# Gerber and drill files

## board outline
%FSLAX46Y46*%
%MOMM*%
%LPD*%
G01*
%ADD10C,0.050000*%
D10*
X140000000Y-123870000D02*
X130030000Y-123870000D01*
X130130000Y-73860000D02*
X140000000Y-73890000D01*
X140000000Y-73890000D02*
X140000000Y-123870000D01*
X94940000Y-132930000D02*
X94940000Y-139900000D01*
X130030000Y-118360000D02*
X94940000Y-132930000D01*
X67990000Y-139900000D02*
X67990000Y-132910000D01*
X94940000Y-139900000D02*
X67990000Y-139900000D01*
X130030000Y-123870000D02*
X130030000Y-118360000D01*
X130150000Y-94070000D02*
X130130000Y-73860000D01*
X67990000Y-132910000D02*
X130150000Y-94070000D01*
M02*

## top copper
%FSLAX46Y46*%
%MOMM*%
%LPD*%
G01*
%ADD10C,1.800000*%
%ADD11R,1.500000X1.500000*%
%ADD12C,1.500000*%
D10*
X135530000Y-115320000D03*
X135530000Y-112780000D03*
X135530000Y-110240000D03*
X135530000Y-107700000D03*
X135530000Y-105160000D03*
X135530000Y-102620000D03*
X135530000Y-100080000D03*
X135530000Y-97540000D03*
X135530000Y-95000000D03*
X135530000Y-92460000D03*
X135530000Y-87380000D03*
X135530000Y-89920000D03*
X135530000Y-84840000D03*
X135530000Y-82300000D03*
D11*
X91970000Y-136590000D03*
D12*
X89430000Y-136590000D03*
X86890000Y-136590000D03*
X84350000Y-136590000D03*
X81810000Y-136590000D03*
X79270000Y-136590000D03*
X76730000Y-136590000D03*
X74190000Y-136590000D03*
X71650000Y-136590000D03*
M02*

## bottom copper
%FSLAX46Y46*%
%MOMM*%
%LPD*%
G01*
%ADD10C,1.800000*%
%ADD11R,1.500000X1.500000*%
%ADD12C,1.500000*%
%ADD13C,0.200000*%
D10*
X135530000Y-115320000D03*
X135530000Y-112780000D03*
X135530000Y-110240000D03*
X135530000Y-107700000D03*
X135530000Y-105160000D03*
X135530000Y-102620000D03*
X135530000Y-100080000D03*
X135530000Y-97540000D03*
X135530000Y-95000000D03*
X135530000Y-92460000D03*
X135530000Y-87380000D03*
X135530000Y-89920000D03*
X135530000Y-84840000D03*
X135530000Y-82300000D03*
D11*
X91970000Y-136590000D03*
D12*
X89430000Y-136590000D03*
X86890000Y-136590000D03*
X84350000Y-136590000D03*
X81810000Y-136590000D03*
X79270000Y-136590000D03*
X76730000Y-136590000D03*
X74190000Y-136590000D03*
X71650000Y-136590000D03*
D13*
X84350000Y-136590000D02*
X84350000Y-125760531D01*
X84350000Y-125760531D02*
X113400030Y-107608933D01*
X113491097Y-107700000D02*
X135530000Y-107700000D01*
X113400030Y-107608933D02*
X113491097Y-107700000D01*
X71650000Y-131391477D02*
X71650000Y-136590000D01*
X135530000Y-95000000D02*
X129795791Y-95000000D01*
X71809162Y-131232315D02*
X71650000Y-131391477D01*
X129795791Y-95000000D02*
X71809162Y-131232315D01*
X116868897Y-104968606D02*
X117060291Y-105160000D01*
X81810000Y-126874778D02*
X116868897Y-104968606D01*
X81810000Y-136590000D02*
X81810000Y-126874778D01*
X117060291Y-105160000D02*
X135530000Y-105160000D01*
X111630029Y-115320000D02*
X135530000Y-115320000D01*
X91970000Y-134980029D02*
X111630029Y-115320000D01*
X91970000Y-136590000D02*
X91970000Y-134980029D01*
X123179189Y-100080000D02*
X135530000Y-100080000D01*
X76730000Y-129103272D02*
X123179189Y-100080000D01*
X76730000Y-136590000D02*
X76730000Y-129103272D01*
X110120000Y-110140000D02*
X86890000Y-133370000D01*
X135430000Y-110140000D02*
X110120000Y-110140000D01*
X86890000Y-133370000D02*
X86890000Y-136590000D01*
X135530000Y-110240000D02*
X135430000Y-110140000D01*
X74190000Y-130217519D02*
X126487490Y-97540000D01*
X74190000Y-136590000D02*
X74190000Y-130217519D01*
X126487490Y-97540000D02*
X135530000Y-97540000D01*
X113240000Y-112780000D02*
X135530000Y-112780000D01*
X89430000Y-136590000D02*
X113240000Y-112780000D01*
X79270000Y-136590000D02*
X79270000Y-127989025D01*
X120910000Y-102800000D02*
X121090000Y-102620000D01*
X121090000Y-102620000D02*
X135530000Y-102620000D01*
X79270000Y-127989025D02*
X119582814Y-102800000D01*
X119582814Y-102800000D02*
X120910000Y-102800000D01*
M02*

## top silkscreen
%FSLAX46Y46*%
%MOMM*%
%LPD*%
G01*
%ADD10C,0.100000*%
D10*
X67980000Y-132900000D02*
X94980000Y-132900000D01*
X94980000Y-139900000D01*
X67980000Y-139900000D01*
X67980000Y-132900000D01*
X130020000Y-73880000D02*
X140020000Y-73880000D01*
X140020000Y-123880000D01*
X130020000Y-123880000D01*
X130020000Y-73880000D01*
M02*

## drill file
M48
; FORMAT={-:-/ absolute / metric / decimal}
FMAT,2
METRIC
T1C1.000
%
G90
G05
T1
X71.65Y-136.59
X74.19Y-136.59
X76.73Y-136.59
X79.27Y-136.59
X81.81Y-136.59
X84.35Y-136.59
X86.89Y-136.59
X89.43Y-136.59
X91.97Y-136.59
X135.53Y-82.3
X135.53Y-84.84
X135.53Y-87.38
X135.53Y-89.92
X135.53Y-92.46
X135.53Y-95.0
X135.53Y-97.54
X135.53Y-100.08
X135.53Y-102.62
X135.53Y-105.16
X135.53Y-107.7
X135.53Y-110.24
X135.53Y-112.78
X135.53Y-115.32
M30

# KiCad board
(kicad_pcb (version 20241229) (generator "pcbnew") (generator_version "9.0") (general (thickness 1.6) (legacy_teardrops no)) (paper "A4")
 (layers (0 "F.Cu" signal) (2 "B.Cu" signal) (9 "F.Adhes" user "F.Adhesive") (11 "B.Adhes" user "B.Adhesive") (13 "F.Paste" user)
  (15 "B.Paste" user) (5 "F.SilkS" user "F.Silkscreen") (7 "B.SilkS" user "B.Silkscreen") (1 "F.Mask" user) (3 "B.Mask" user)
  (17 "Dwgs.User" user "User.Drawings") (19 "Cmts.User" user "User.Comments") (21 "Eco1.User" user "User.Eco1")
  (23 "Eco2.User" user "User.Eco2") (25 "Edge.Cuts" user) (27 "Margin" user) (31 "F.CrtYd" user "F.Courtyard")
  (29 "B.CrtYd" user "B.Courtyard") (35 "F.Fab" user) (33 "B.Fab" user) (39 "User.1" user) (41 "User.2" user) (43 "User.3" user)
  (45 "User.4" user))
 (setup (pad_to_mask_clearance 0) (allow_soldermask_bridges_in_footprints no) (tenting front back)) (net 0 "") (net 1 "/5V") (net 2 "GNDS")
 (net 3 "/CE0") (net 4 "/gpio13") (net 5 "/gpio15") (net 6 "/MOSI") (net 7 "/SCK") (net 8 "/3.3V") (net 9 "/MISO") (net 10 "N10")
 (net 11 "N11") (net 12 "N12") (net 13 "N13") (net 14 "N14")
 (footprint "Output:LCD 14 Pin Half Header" (layer "F.Cu") (at 133.02 73.88)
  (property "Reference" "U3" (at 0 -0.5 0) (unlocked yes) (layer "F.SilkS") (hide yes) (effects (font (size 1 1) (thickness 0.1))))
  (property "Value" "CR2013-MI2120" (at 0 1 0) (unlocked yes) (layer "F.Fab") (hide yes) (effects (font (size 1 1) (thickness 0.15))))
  (fp_rect (start -3 0) (end 7 50) (stroke (width 0.1) (type solid)) (fill no) (layer "F.SilkS"))
  (pad "1" thru_hole circle (at 2.51 41.44 180) (size 1.8 1.8) (drill 1) (layers "*.Cu" "*.Mask") (remove_unused_layers no) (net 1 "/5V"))
  (pad "2" thru_hole circle (at 2.51 38.9 180) (size 1.8 1.8) (drill 1) (layers "*.Cu" "*.Mask") (remove_unused_layers no) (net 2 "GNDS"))
  (pad "3" thru_hole circle (at 2.51 36.36 180) (size 1.8 1.8) (drill 1) (layers "*.Cu" "*.Mask") (remove_unused_layers no) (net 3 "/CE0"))
  (pad "4" thru_hole circle (at 2.51 33.82 180) (size 1.8 1.8) (drill 1) (layers "*.Cu" "*.Mask") (remove_unused_layers no)
   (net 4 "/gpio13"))
  (pad "5" thru_hole circle (at 2.51 31.28 180) (size 1.8 1.8) (drill 1) (layers "*.Cu" "*.Mask") (remove_unused_layers no)
   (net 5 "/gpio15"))
  (pad "6" thru_hole circle (at 2.51 28.74 180) (size 1.8 1.8) (drill 1) (layers "*.Cu" "*.Mask") (remove_unused_layers no) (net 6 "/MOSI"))
  (pad "7" thru_hole circle (at 2.51 26.2 180) (size 1.8 1.8) (drill 1) (layers "*.Cu" "*.Mask") (remove_unused_layers no) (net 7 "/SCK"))
  (pad "8" thru_hole circle (at 2.51 23.66 180) (size 1.8 1.8) (drill 1) (layers "*.Cu" "*.Mask") (remove_unused_layers no) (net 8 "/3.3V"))
  (pad "9" thru_hole circle (at 2.51 21.12 180) (size 1.8 1.8) (drill 1) (layers "*.Cu" "*.Mask") (remove_unused_layers no) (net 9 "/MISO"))
  (pad "10" thru_hole circle (at 2.51 18.58 180) (size 1.8 1.8) (drill 1) (layers "*.Cu" "*.Mask") (remove_unused_layers no) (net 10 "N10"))
  (pad "11" thru_hole circle (at 2.51 13.5 180) (size 1.8 1.8) (drill 1) (layers "*.Cu" "*.Mask") (remove_unused_layers no) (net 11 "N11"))
  (pad "12" thru_hole circle (at 2.51 16.04 180) (size 1.8 1.8) (drill 1) (layers "*.Cu" "*.Mask") (remove_unused_layers no) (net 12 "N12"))
  (pad "13" thru_hole circle (at 2.51 10.96 180) (size 1.8 1.8) (drill 1) (layers "*.Cu" "*.Mask") (remove_unused_layers no) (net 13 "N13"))
  (pad "14" thru_hole circle (at 2.51 8.42 180) (size 1.8 1.8) (drill 1) (layers "*.Cu" "*.Mask") (remove_unused_layers no) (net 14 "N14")))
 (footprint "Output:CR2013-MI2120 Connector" (layer "F.Cu") (at 91.97 136.59 -90)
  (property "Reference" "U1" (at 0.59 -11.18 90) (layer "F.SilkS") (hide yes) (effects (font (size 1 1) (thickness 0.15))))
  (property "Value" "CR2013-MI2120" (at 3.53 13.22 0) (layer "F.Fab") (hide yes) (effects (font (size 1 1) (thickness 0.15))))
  (pad "1" thru_hole rect (at 0 0 270) (size 1.5 1.5) (drill 1) (layers "*.Cu" "*.Mask") (remove_unused_layers no) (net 1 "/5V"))
  (pad "2" thru_hole circle (at 0 2.54 270) (size 1.5 1.5) (drill 1) (layers "*.Cu" "*.Mask") (remove_unused_layers no) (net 2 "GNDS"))
  (pad "3" thru_hole circle (at 0 5.08 270) (size 1.5 1.5) (drill 1) (layers "*.Cu" "*.Mask") (remove_unused_layers no) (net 3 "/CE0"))
  (pad "4" thru_hole circle (at 0 7.62 270) (size 1.5 1.5) (drill 1) (layers "*.Cu" "*.Mask") (remove_unused_layers no) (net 4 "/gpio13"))
  (pad "5" thru_hole circle (at 0 10.16 270) (size 1.5 1.5) (drill 1) (layers "*.Cu" "*.Mask") (remove_unused_layers no) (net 5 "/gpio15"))
  (pad "6" thru_hole circle (at 0 12.7 270) (size 1.5 1.5) (drill 1) (layers "*.Cu" "*.Mask") (remove_unused_layers no) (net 6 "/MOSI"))
  (pad "7" thru_hole circle (at 0 15.24 270) (size 1.5 1.5) (drill 1) (layers "*.Cu" "*.Mask") (remove_unused_layers no) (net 7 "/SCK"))
  (pad "8" thru_hole circle (at 0 17.78 270) (size 1.5 1.5) (drill 1) (layers "*.Cu" "*.Mask") (remove_unused_layers no) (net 8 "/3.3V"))
  (pad "9" thru_hole circle (at 0 20.32 270) (size 1.5 1.5) (drill 1) (layers "*.Cu" "*.Mask") (remove_unused_layers no) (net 9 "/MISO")))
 (gr_rect (start 67.98 132.9) (end 94.98 139.9) (stroke (width 0.1) (type solid)) (fill no) (layer "F.SilkS"))
 (gr_line (start 140 123.87) (end 130.03 123.87) (stroke (width 0.05) (type default)) (layer "Edge.Cuts"))
 (gr_line (start 130.13 73.86) (end 140 73.89) (stroke (width 0.05) (type default)) (layer "Edge.Cuts"))
 (gr_line (start 140 73.89) (end 140 123.87) (stroke (width 0.05) (type default)) (layer "Edge.Cuts"))
 (gr_line (start 94.94 132.93) (end 94.94 139.9) (stroke (width 0.05) (type default)) (layer "Edge.Cuts"))
 (gr_line (start 130.03 118.36) (end 94.94 132.93) (stroke (width 0.05) (type default)) (layer "Edge.Cuts"))
 (gr_line (start 67.99 139.9) (end 67.99 132.91) (stroke (width 0.05) (type default)) (layer "Edge.Cuts"))
 (gr_line (start 94.94 139.9) (end 67.99 139.9) (stroke (width 0.05) (type default)) (layer "Edge.Cuts"))
 (gr_line (start 130.03 123.87) (end 130.03 118.36) (stroke (width 0.05) (type default)) (layer "Edge.Cuts"))
 (gr_line (start 130.15 94.07) (end 130.13 73.86) (stroke (width 0.05) (type default)) (layer "Edge.Cuts"))
 (gr_line (start 67.99 132.91) (end 130.15 94.07) (stroke (width 0.05) (type default)) (layer "Edge.Cuts"))
 (segment (start 84.35 136.59) (end 84.35 125.760531) (width 0.2) (layer "B.Cu") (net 4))
 (segment (start 84.35 125.760531) (end 113.40003 107.608933) (width 0.2) (layer "B.Cu") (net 4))
 (segment (start 113.491097 107.7) (end 135.53 107.7) (width 0.2) (layer "B.Cu") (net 4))
 (segment (start 113.40003 107.608933) (end 113.491097 107.7) (width 0.2) (layer "B.Cu") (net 4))
 (segment (start 71.65 131.391477) (end 71.65 136.59) (width 0.2) (layer "B.Cu") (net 9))
 (segment (start 135.53 95) (end 129.795791 95) (width 0.2) (layer "B.Cu") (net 9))
 (segment (start 71.809162 131.232315) (end 71.65 131.391477) (width 0.2) (layer "B.Cu") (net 9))
 (segment (start 129.795791 95) (end 71.809162 131.232315) (width 0.2) (layer "B.Cu") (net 9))
 (segment (start 116.868897 104.968606) (end 117.060291 105.16) (width 0.2) (layer "B.Cu") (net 5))
 (segment (start 81.81 126.874778) (end 116.868897 104.968606) (width 0.2) (layer "B.Cu") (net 5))
 (segment (start 81.81 136.59) (end 81.81 126.874778) (width 0.2) (layer "B.Cu") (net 5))
 (segment (start 117.060291 105.16) (end 135.53 105.16) (width 0.2) (layer "B.Cu") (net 5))
 (segment (start 111.630029 115.32) (end 135.53 115.32) (width 0.2) (layer "B.Cu") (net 1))
 (segment (start 91.97 134.980029) (end 111.630029 115.32) (width 0.2) (layer "B.Cu") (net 1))
 (segment (start 91.97 136.59) (end 91.97 134.980029) (width 0.2) (layer "B.Cu") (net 1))
 (segment (start 123.179189 100.08) (end 135.53 100.08) (width 0.2) (layer "B.Cu") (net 7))
 (segment (start 76.73 129.103272) (end 123.179189 100.08) (width 0.2) (layer "B.Cu") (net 7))
 (segment (start 76.73 136.59) (end 76.73 129.103272) (width 0.2) (layer "B.Cu") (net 7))
 (segment (start 110.12 110.14) (end 86.89 133.37) (width 0.2) (layer "B.Cu") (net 3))
 (segment (start 135.43 110.14) (end 110.12 110.14) (width 0.2) (layer "B.Cu") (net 3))
 (segment (start 86.89 133.37) (end 86.89 136.59) (width 0.2) (layer "B.Cu") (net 3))
 (segment (start 135.53 110.24) (end 135.43 110.14) (width 0.2) (layer "B.Cu") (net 3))
 (segment (start 74.19 130.217519) (end 126.48749 97.54) (width 0.2) (layer "B.Cu") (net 8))
 (segment (start 74.19 136.59) (end 74.19 130.217519) (width 0.2) (layer "B.Cu") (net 8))
 (segment (start 126.48749 97.54) (end 135.53 97.54) (width 0.2) (layer "B.Cu") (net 8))
 (segment (start 113.24 112.78) (end 135.53 112.78) (width 0.2) (layer "B.Cu") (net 2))
 (segment (start 89.43 136.59) (end 113.24 112.78) (width 0.2) (layer "B.Cu") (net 2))
 (segment (start 79.27 136.59) (end 79.27 127.989025) (width 0.2) (layer "B.Cu") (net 6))
 (segment (start 120.91 102.8) (end 121.09 102.62) (width 0.2) (layer "B.Cu") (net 6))
 (segment (start 121.09 102.62) (end 135.53 102.62) (width 0.2) (layer "B.Cu") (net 6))
 (segment (start 79.27 127.989025) (end 119.582814 102.8) (width 0.2) (layer "B.Cu") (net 6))
 (segment (start 119.582814 102.8) (end 120.91 102.8) (width 0.2) (layer "B.Cu") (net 6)))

